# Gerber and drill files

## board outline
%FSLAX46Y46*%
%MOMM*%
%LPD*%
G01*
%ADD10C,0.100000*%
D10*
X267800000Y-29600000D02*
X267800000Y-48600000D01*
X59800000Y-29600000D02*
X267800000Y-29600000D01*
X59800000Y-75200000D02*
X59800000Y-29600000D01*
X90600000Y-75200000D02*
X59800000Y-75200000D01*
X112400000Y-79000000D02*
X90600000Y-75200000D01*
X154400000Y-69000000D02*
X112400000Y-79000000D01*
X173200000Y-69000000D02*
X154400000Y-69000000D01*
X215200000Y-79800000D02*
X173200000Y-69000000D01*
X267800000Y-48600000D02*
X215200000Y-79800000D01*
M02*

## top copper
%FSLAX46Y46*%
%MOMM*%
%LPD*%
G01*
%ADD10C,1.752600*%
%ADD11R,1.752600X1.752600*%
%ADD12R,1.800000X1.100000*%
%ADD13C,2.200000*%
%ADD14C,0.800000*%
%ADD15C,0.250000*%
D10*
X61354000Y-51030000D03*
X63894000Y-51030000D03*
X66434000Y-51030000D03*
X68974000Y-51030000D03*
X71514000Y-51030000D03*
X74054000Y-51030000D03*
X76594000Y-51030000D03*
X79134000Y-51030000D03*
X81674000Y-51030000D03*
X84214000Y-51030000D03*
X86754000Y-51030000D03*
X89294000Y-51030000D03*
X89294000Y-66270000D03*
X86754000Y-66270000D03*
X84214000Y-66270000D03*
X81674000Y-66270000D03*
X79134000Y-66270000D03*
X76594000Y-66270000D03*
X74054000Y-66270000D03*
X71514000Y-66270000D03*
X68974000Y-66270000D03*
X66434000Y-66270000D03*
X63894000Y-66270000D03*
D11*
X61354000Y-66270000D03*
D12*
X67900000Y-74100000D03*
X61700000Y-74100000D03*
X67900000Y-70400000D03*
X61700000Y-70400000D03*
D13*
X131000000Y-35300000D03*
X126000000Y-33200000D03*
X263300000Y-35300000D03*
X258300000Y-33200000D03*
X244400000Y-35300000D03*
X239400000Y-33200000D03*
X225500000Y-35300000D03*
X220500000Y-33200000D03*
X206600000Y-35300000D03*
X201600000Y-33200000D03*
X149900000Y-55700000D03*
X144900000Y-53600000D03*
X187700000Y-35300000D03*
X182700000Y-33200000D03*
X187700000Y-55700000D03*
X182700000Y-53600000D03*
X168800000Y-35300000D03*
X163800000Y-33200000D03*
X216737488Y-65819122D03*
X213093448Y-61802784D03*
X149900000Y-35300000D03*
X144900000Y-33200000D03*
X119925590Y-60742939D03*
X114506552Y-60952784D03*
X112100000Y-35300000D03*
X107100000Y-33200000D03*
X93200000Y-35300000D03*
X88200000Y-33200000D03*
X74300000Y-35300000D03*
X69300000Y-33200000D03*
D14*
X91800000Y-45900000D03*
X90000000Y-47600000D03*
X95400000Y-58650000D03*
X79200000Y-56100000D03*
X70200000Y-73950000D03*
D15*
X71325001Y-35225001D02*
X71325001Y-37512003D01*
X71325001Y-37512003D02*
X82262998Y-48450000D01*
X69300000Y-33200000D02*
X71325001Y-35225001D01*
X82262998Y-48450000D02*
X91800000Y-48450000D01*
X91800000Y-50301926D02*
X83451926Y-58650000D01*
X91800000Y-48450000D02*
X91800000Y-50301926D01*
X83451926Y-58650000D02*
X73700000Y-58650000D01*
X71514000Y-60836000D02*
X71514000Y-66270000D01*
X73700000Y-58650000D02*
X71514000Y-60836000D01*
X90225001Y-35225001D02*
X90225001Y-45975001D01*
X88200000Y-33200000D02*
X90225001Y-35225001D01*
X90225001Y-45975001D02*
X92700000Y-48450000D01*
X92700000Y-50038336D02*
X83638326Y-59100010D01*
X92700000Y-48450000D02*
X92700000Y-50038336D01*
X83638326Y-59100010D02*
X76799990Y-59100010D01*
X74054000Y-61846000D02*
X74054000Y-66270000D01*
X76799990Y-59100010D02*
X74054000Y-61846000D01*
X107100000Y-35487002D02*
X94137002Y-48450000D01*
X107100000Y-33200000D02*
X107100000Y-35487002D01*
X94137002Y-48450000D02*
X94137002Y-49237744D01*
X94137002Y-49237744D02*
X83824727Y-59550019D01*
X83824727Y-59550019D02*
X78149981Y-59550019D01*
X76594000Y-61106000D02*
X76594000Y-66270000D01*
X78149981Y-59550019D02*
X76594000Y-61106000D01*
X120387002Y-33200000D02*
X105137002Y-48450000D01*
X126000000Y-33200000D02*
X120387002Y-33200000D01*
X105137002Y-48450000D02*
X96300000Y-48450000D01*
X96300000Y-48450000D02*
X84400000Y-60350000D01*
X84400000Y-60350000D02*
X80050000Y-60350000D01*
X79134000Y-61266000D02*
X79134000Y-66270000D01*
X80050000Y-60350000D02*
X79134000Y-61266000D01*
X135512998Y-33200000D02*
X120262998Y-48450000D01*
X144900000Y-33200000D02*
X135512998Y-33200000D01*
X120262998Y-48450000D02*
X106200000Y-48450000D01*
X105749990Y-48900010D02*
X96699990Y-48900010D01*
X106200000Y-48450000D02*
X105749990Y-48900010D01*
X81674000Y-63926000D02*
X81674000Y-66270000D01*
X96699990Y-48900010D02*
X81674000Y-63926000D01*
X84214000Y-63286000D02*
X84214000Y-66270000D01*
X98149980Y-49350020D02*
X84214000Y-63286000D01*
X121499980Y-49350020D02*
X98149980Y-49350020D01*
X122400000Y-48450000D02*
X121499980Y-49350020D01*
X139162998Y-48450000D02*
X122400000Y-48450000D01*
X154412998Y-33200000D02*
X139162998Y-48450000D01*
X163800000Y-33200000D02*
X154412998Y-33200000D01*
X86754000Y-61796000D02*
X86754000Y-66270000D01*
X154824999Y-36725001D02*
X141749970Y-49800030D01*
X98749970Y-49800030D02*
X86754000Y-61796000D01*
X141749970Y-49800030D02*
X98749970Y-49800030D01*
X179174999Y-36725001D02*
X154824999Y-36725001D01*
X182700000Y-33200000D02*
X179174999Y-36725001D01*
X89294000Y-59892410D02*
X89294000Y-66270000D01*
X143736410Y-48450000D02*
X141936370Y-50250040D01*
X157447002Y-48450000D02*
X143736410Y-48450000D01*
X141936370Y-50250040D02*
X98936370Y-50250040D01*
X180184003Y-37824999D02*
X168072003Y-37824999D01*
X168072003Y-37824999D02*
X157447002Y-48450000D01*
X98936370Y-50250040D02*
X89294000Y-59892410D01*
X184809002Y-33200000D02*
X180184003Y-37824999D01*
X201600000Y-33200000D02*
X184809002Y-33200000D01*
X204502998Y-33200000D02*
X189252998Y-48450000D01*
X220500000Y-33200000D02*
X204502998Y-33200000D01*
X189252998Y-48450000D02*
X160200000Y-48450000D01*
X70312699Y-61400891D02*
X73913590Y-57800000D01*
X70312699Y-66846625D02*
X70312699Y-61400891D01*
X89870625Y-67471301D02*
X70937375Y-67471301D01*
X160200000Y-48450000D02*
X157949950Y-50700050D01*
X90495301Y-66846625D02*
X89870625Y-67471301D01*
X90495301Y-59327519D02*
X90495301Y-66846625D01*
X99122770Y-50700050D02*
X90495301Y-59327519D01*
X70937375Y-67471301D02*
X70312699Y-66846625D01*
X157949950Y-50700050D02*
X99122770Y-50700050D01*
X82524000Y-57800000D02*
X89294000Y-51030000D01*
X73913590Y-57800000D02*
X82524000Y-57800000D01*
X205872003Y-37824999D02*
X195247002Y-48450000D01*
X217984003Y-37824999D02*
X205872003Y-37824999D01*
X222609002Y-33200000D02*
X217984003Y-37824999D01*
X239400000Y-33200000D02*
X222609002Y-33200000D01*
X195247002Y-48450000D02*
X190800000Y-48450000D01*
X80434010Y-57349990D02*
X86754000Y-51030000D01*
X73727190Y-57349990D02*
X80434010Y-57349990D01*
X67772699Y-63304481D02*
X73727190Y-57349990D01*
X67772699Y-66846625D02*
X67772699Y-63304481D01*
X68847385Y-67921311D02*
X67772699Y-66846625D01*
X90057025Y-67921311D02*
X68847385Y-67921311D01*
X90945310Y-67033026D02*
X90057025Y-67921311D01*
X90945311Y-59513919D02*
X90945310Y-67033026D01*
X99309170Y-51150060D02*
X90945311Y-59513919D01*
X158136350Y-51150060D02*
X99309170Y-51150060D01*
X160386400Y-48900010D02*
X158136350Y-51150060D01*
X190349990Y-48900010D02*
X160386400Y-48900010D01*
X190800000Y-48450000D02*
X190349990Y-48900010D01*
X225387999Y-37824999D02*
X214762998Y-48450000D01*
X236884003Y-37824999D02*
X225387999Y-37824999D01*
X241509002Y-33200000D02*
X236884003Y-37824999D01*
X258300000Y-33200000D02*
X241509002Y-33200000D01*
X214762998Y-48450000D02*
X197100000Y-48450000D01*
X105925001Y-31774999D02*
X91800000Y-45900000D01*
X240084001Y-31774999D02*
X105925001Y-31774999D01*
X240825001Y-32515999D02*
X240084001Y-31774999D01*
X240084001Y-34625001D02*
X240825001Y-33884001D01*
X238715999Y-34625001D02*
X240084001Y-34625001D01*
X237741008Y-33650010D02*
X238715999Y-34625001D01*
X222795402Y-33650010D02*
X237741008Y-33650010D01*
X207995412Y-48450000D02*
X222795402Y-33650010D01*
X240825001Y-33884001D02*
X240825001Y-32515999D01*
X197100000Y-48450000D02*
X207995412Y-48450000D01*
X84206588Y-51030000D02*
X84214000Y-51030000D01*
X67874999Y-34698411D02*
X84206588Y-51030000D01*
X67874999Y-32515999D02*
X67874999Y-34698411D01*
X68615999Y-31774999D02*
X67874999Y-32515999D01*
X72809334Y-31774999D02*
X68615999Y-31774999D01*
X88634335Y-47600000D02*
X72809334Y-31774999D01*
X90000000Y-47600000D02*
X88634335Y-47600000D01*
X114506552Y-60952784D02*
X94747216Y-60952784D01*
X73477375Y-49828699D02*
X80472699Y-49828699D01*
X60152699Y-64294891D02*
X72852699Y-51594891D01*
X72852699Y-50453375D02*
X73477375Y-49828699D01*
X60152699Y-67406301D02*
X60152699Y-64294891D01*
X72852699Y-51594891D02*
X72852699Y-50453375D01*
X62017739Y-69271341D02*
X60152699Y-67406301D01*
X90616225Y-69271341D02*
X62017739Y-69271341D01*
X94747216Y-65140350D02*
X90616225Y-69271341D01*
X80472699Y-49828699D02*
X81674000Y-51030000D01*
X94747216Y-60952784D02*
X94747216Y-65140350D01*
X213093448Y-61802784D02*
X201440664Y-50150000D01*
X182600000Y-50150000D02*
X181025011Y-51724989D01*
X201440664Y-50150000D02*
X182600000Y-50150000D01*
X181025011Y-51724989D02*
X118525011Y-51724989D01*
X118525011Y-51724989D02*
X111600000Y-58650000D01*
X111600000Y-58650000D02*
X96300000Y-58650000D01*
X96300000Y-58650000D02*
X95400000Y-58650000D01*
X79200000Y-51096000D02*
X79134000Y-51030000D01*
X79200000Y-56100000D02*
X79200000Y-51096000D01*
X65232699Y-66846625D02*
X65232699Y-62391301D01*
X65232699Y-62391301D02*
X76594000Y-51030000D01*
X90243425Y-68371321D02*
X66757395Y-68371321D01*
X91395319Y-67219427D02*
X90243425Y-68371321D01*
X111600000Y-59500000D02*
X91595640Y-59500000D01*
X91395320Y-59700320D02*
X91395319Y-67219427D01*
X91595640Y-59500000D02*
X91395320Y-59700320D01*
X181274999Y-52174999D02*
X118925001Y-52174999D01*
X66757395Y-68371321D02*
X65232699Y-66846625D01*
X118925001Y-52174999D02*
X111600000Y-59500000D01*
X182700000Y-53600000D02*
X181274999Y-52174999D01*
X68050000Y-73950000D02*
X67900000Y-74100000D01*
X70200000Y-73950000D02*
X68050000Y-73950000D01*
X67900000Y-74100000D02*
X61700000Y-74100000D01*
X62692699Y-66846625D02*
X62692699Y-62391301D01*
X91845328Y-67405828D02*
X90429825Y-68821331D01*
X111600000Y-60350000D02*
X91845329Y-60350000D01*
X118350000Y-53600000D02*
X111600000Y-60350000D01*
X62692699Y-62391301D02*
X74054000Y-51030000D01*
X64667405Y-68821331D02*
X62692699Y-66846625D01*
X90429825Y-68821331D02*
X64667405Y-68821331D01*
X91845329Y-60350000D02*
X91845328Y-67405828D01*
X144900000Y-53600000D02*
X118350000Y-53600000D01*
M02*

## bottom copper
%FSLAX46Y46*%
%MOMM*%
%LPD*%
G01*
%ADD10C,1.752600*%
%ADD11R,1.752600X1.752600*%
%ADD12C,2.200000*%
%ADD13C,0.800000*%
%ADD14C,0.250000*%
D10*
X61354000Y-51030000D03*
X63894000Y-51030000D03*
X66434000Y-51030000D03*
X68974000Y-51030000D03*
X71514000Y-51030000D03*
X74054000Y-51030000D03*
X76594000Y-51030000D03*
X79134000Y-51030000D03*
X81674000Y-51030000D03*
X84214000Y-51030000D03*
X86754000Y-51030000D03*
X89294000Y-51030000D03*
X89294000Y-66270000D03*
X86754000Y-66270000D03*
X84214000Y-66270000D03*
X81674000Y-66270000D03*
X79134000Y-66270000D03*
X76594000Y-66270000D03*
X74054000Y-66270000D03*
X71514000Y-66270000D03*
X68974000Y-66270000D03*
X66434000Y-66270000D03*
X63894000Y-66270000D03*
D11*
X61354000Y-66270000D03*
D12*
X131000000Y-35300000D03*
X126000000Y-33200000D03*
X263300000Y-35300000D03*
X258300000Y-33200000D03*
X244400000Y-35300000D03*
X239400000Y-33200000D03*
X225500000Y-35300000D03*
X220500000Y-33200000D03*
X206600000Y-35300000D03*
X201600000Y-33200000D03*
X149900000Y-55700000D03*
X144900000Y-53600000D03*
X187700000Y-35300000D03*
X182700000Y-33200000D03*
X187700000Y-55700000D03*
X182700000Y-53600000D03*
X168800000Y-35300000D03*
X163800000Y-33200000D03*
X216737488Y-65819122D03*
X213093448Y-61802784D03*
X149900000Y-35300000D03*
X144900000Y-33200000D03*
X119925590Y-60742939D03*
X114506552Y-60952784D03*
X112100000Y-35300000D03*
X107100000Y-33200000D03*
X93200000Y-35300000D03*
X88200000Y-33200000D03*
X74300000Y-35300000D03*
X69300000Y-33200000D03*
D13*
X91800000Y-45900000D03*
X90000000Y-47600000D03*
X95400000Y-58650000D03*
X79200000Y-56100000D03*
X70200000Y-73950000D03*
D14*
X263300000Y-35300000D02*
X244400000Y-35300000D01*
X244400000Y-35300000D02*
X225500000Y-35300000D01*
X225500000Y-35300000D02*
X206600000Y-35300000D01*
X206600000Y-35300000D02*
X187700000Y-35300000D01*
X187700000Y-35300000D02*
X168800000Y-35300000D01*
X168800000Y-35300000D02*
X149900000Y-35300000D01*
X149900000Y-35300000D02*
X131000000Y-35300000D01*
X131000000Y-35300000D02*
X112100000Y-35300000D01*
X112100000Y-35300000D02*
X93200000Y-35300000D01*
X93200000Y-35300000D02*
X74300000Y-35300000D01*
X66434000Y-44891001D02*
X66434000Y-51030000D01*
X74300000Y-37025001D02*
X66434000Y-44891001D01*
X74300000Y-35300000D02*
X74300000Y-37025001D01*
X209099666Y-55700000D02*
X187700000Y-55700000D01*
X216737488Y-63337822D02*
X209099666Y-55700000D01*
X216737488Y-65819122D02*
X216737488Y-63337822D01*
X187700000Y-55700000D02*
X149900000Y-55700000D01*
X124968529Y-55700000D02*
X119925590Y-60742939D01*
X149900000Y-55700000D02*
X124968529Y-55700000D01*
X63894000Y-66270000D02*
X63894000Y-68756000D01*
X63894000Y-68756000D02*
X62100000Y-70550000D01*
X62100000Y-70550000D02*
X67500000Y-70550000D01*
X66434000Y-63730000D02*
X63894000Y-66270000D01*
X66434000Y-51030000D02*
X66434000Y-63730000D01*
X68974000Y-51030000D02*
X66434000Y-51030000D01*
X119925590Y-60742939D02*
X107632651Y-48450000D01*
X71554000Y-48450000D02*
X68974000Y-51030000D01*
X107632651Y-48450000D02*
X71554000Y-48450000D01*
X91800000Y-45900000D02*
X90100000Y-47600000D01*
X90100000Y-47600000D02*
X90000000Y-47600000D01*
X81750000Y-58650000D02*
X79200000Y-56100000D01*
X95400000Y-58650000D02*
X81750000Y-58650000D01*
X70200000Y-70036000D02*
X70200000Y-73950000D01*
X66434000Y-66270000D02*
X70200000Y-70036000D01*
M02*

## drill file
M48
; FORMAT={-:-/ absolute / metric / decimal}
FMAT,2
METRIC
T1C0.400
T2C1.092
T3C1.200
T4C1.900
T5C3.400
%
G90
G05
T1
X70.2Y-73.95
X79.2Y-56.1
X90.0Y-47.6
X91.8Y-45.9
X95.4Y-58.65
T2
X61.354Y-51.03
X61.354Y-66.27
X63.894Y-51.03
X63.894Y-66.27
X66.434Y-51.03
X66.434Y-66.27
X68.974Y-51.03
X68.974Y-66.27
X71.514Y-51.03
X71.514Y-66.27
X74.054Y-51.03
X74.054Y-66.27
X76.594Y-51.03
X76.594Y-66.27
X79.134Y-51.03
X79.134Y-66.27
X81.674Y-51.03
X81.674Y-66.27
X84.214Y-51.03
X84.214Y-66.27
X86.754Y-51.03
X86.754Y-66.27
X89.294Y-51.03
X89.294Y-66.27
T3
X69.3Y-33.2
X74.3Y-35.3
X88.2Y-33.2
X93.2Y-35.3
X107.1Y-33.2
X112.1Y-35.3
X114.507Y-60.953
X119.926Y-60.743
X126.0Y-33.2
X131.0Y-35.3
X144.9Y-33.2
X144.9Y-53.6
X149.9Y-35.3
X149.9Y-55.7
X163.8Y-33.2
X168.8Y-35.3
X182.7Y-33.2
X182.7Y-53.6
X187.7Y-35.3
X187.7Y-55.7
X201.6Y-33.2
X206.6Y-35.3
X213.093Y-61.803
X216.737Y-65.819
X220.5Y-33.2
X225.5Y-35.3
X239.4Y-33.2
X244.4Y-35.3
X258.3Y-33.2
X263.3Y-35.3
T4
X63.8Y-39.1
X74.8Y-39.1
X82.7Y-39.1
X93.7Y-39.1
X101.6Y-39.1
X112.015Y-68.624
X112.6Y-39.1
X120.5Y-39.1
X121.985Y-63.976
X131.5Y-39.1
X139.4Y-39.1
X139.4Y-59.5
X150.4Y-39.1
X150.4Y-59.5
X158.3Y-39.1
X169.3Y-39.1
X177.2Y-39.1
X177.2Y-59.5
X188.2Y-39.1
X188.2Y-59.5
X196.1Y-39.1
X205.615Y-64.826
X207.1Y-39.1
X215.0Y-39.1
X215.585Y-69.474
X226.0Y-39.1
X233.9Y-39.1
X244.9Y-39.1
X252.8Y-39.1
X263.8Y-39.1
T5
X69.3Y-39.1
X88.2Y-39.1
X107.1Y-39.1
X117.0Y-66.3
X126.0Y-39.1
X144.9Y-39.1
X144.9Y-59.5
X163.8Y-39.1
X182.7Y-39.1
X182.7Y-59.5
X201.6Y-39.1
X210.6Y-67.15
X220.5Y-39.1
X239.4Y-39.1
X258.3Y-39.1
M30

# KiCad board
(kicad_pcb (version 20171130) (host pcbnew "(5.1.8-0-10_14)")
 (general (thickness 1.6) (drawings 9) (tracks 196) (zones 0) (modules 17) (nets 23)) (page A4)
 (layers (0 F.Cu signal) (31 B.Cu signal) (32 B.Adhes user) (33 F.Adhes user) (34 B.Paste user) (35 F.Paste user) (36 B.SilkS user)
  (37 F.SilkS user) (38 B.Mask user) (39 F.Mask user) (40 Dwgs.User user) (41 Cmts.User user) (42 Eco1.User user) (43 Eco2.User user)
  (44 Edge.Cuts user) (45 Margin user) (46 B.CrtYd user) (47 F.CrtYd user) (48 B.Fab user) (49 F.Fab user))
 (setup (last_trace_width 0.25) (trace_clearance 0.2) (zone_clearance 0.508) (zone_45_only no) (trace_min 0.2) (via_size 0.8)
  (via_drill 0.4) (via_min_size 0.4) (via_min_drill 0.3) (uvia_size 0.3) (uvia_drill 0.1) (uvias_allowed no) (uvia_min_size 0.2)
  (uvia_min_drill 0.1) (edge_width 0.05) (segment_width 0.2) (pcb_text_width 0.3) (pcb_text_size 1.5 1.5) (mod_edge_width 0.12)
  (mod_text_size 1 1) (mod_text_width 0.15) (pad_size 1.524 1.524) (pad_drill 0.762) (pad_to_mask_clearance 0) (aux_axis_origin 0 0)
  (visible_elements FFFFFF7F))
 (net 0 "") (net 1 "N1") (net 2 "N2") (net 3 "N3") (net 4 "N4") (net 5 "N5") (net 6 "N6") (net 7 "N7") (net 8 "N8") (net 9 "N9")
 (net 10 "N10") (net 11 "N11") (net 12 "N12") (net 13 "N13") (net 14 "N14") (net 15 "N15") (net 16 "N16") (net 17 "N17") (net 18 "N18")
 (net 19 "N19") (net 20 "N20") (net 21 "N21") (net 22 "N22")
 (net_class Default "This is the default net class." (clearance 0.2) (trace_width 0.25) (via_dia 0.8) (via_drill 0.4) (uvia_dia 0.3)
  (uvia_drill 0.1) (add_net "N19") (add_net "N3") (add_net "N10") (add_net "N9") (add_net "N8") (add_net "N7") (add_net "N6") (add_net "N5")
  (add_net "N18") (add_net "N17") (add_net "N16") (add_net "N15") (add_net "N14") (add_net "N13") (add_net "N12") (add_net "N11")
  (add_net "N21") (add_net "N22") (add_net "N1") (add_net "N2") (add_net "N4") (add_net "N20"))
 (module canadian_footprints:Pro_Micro (layer F.Cu) (at 73.8 58.65 90)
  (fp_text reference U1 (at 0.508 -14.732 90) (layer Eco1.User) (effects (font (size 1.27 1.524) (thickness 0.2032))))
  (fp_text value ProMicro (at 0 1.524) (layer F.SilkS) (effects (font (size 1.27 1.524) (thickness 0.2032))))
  (pad 13 thru_hole circle (at 7.62 -12.446) (size 1.7526 1.7526) (drill 1.0922) (layers *.Cu *.SilkS *.Mask) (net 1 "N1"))
  (pad 14 thru_hole circle (at 7.62 -9.906) (size 1.7526 1.7526) (drill 1.0922) (layers *.Cu *.SilkS *.Mask) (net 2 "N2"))
  (pad 15 thru_hole circle (at 7.62 -7.366) (size 1.7526 1.7526) (drill 1.0922) (layers *.Cu *.SilkS *.Mask) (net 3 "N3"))
  (pad 16 thru_hole circle (at 7.62 -4.826) (size 1.7526 1.7526) (drill 1.0922) (layers *.Cu *.SilkS *.Mask) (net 3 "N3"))
  (pad 17 thru_hole circle (at 7.62 -2.286) (size 1.7526 1.7526) (drill 1.0922) (layers *.Cu *.SilkS *.Mask) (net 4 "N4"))
  (pad 18 thru_hole circle (at 7.62 0.254) (size 1.7526 1.7526) (drill 1.0922) (layers *.Cu *.SilkS *.Mask) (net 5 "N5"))
  (pad 19 thru_hole circle (at 7.62 2.794) (size 1.7526 1.7526) (drill 1.0922) (layers *.Cu *.SilkS *.Mask) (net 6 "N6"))
  (pad 20 thru_hole circle (at 7.62 5.334) (size 1.7526 1.7526) (drill 1.0922) (layers *.Cu *.SilkS *.Mask) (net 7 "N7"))
  (pad 21 thru_hole circle (at 7.62 7.874) (size 1.7526 1.7526) (drill 1.0922) (layers *.Cu *.SilkS *.Mask) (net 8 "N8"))
  (pad 22 thru_hole circle (at 7.62 10.414) (size 1.7526 1.7526) (drill 1.0922) (layers *.Cu *.SilkS *.Mask) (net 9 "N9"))
  (pad 23 thru_hole circle (at 7.62 12.954) (size 1.7526 1.7526) (drill 1.0922) (layers *.Cu *.SilkS *.Mask) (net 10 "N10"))
  (pad 24 thru_hole circle (at 7.62 15.494) (size 1.7526 1.7526) (drill 1.0922) (layers *.Cu *.SilkS *.Mask) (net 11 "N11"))
  (pad 12 thru_hole circle (at -7.62 15.494) (size 1.7526 1.7526) (drill 1.0922) (layers *.Cu *.SilkS *.Mask) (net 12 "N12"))
  (pad 11 thru_hole circle (at -7.62 12.954) (size 1.7526 1.7526) (drill 1.0922) (layers *.Cu *.SilkS *.Mask) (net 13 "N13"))
  (pad 10 thru_hole circle (at -7.62 10.414) (size 1.7526 1.7526) (drill 1.0922) (layers *.Cu *.SilkS *.Mask) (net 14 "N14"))
  (pad 9 thru_hole circle (at -7.62 7.874) (size 1.7526 1.7526) (drill 1.0922) (layers *.Cu *.SilkS *.Mask) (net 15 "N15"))
  (pad 8 thru_hole circle (at -7.62 5.334) (size 1.7526 1.7526) (drill 1.0922) (layers *.Cu *.SilkS *.Mask) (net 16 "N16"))
  (pad 7 thru_hole circle (at -7.62 2.794) (size 1.7526 1.7526) (drill 1.0922) (layers *.Cu *.SilkS *.Mask) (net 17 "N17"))
  (pad 6 thru_hole circle (at -7.62 0.254) (size 1.7526 1.7526) (drill 1.0922) (layers *.Cu *.SilkS *.Mask) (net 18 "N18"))
  (pad 5 thru_hole circle (at -7.62 -2.286) (size 1.7526 1.7526) (drill 1.0922) (layers *.Cu *.SilkS *.Mask) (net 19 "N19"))
  (pad 4 thru_hole circle (at -7.62 -4.826) (size 1.7526 1.7526) (drill 1.0922) (layers *.Cu *.SilkS *.Mask) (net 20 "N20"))
  (pad 3 thru_hole circle (at -7.62 -7.366) (size 1.7526 1.7526) (drill 1.0922) (layers *.Cu *.SilkS *.Mask) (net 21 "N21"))
  (pad 2 thru_hole circle (at -7.62 -9.906) (size 1.7526 1.7526) (drill 1.0922) (layers *.Cu *.SilkS *.Mask) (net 3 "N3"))
  (pad 1 thru_hole rect (at -7.62 -12.446) (size 1.7526 1.7526) (drill 1.0922) (layers *.Cu *.SilkS *.Mask) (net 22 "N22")))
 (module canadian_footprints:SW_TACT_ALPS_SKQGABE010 (layer F.Cu) (at 64.8 72.25)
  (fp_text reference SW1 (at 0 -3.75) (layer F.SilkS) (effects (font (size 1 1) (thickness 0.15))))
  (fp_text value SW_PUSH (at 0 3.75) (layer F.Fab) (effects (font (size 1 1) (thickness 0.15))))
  (pad 2 smd rect (at 3.1 1.85) (size 1.8 1.1) (layers F.Cu F.Paste F.Mask) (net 21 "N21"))
  (pad 2 smd rect (at -3.1 1.85) (size 1.8 1.1) (layers F.Cu F.Paste F.Mask) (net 21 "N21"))
  (pad 1 smd rect (at 3.1 -1.85) (size 1.8 1.1) (layers F.Cu F.Paste F.Mask) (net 3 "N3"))
  (pad 1 smd rect (at -3.1 -1.85) (size 1.8 1.1) (layers F.Cu F.Paste F.Mask) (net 3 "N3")))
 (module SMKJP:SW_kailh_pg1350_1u (layer F.Cu) (at 126 39.1)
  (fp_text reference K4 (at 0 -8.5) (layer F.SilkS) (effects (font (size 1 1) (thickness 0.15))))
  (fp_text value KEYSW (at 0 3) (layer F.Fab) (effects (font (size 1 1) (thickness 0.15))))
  (pad 2 thru_hole circle (at 5 -3.8) (size 2.2 2.2) (drill 1.2) (layers *.Cu *.Mask) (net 3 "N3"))
  (pad 1 thru_hole circle (at 0 -5.9) (size 2.2 2.2) (drill 1.2) (layers *.Cu *.Mask) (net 16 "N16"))
  (pad "" np_thru_hole circle (at 5.5 0) (size 1.9 1.9) (drill 1.9) (layers *.Cu *.Mask))
  (pad "" np_thru_hole circle (at -5.5 0) (size 1.9 1.9) (drill 1.9) (layers *.Cu *.Mask))
  (pad "" np_thru_hole circle (at 0 0) (size 3.4 3.4) (drill 3.4) (layers *.Cu *.Mask)))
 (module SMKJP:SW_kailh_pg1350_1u (layer F.Cu) (at 258.3 39.1)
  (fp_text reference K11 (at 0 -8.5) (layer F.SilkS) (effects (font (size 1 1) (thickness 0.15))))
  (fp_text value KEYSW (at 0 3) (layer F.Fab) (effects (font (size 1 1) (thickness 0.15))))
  (pad 2 thru_hole circle (at 5 -3.8) (size 2.2 2.2) (drill 1.2) (layers *.Cu *.Mask) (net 3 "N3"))
  (pad 1 thru_hole circle (at 0 -5.9) (size 2.2 2.2) (drill 1.2) (layers *.Cu *.Mask) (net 9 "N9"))
  (pad "" np_thru_hole circle (at 5.5 0) (size 1.9 1.9) (drill 1.9) (layers *.Cu *.Mask))
  (pad "" np_thru_hole circle (at -5.5 0) (size 1.9 1.9) (drill 1.9) (layers *.Cu *.Mask))
  (pad "" np_thru_hole circle (at 0 0) (size 3.4 3.4) (drill 3.4) (layers *.Cu *.Mask)))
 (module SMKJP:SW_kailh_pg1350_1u (layer F.Cu) (at 239.4 39.1)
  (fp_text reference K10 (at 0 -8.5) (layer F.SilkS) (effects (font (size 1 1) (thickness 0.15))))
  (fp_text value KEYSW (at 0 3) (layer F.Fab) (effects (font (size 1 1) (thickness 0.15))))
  (pad 2 thru_hole circle (at 5 -3.8) (size 2.2 2.2) (drill 1.2) (layers *.Cu *.Mask) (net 3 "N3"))
  (pad 1 thru_hole circle (at 0 -5.9) (size 2.2 2.2) (drill 1.2) (layers *.Cu *.Mask) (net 10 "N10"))
  (pad "" np_thru_hole circle (at 5.5 0) (size 1.9 1.9) (drill 1.9) (layers *.Cu *.Mask))
  (pad "" np_thru_hole circle (at -5.5 0) (size 1.9 1.9) (drill 1.9) (layers *.Cu *.Mask))
  (pad "" np_thru_hole circle (at 0 0) (size 3.4 3.4) (drill 3.4) (layers *.Cu *.Mask)))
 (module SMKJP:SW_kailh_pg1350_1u (layer F.Cu) (at 220.5 39.1)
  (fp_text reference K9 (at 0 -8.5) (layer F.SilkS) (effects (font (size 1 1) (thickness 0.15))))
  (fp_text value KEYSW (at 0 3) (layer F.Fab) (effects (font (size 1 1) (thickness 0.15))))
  (pad 2 thru_hole circle (at 5 -3.8) (size 2.2 2.2) (drill 1.2) (layers *.Cu *.Mask) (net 3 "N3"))
  (pad 1 thru_hole circle (at 0 -5.9) (size 2.2 2.2) (drill 1.2) (layers *.Cu *.Mask) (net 11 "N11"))
  (pad "" np_thru_hole circle (at 5.5 0) (size 1.9 1.9) (drill 1.9) (layers *.Cu *.Mask))
  (pad "" np_thru_hole circle (at -5.5 0) (size 1.9 1.9) (drill 1.9) (layers *.Cu *.Mask))
  (pad "" np_thru_hole circle (at 0 0) (size 3.4 3.4) (drill 3.4) (layers *.Cu *.Mask)))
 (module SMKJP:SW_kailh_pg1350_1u (layer F.Cu) (at 201.6 39.1)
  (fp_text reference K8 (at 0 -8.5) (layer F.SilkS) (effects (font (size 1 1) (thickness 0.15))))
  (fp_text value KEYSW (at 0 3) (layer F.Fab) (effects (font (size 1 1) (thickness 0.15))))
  (pad 2 thru_hole circle (at 5 -3.8) (size 2.2 2.2) (drill 1.2) (layers *.Cu *.Mask) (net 3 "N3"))
  (pad 1 thru_hole circle (at 0 -5.9) (size 2.2 2.2) (drill 1.2) (layers *.Cu *.Mask) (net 12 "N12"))
  (pad "" np_thru_hole circle (at 5.5 0) (size 1.9 1.9) (drill 1.9) (layers *.Cu *.Mask))
  (pad "" np_thru_hole circle (at -5.5 0) (size 1.9 1.9) (drill 1.9) (layers *.Cu *.Mask))
  (pad "" np_thru_hole circle (at 0 0) (size 3.4 3.4) (drill 3.4) (layers *.Cu *.Mask)))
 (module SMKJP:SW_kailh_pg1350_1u (layer F.Cu) (at 144.9 59.5)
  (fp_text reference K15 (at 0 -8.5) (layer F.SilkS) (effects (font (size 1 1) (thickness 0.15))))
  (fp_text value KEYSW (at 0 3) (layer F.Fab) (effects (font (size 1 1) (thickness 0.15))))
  (pad 2 thru_hole circle (at 5 -3.8) (size 2.2 2.2) (drill 1.2) (layers *.Cu *.Mask) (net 3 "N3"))
  (pad 1 thru_hole circle (at 0 -5.9) (size 2.2 2.2) (drill 1.2) (layers *.Cu *.Mask) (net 5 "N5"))
  (pad "" np_thru_hole circle (at 5.5 0) (size 1.9 1.9) (drill 1.9) (layers *.Cu *.Mask))
  (pad "" np_thru_hole circle (at -5.5 0) (size 1.9 1.9) (drill 1.9) (layers *.Cu *.Mask))
  (pad "" np_thru_hole circle (at 0 0) (size 3.4 3.4) (drill 3.4) (layers *.Cu *.Mask)))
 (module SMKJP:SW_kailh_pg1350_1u (layer F.Cu) (at 182.7 39.1)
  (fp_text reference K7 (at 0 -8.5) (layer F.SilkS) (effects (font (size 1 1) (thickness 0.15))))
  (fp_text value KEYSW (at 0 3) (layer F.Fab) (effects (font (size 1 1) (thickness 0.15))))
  (pad 2 thru_hole circle (at 5 -3.8) (size 2.2 2.2) (drill 1.2) (layers *.Cu *.Mask) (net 3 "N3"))
  (pad 1 thru_hole circle (at 0 -5.9) (size 2.2 2.2) (drill 1.2) (layers *.Cu *.Mask) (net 13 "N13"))
  (pad "" np_thru_hole circle (at 5.5 0) (size 1.9 1.9) (drill 1.9) (layers *.Cu *.Mask))
  (pad "" np_thru_hole circle (at -5.5 0) (size 1.9 1.9) (drill 1.9) (layers *.Cu *.Mask))
  (pad "" np_thru_hole circle (at 0 0) (size 3.4 3.4) (drill 3.4) (layers *.Cu *.Mask)))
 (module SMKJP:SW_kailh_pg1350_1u (layer F.Cu) (at 182.7 59.5)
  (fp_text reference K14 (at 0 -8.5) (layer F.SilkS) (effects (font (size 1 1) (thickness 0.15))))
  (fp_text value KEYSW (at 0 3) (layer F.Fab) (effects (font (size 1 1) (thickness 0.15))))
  (pad 2 thru_hole circle (at 5 -3.8) (size 2.2 2.2) (drill 1.2) (layers *.Cu *.Mask) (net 3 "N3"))
  (pad 1 thru_hole circle (at 0 -5.9) (size 2.2 2.2) (drill 1.2) (layers *.Cu *.Mask) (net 6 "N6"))
  (pad "" np_thru_hole circle (at 5.5 0) (size 1.9 1.9) (drill 1.9) (layers *.Cu *.Mask))
  (pad "" np_thru_hole circle (at -5.5 0) (size 1.9 1.9) (drill 1.9) (layers *.Cu *.Mask))
  (pad "" np_thru_hole circle (at 0 0) (size 3.4 3.4) (drill 3.4) (layers *.Cu *.Mask)))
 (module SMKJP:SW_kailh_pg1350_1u (layer F.Cu) (at 163.8 39.1)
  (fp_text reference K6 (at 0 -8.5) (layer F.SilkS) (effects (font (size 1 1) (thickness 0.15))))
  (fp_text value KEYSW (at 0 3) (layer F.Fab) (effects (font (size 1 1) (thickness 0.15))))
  (pad 2 thru_hole circle (at 5 -3.8) (size 2.2 2.2) (drill 1.2) (layers *.Cu *.Mask) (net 3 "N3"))
  (pad 1 thru_hole circle (at 0 -5.9) (size 2.2 2.2) (drill 1.2) (layers *.Cu *.Mask) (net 14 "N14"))
  (pad "" np_thru_hole circle (at 5.5 0) (size 1.9 1.9) (drill 1.9) (layers *.Cu *.Mask))
  (pad "" np_thru_hole circle (at -5.5 0) (size 1.9 1.9) (drill 1.9) (layers *.Cu *.Mask))
  (pad "" np_thru_hole circle (at 0 0) (size 3.4 3.4) (drill 3.4) (layers *.Cu *.Mask)))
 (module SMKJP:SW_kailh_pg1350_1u (layer F.Cu) (at 210.6 67.15 335)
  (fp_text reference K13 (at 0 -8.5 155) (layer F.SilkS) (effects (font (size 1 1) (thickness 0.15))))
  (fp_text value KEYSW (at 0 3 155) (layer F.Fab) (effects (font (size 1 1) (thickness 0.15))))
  (pad 2 thru_hole circle (at 5 -3.8 335) (size 2.2 2.2) (drill 1.2) (layers *.Cu *.Mask) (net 3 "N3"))
  (pad 1 thru_hole circle (at 0 -5.9 335) (size 2.2 2.2) (drill 1.2) (layers *.Cu *.Mask) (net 7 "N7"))
  (pad "" np_thru_hole circle (at 5.5 0 335) (size 1.9 1.9) (drill 1.9) (layers *.Cu *.Mask))
  (pad "" np_thru_hole circle (at -5.5 0 335) (size 1.9 1.9) (drill 1.9) (layers *.Cu *.Mask))
  (pad "" np_thru_hole circle (at 0 0 335) (size 3.4 3.4) (drill 3.4) (layers *.Cu *.Mask)))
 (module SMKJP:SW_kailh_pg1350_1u (layer F.Cu) (at 144.9 39.1)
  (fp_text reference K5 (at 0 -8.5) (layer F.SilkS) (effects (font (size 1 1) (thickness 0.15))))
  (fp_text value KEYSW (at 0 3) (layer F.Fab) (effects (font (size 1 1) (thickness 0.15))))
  (pad 2 thru_hole circle (at 5 -3.8) (size 2.2 2.2) (drill 1.2) (layers *.Cu *.Mask) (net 3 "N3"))
  (pad 1 thru_hole circle (at 0 -5.9) (size 2.2 2.2) (drill 1.2) (layers *.Cu *.Mask) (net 15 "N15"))
  (pad "" np_thru_hole circle (at 5.5 0) (size 1.9 1.9) (drill 1.9) (layers *.Cu *.Mask))
  (pad "" np_thru_hole circle (at -5.5 0) (size 1.9 1.9) (drill 1.9) (layers *.Cu *.Mask))
  (pad "" np_thru_hole circle (at 0 0) (size 3.4 3.4) (drill 3.4) (layers *.Cu *.Mask)))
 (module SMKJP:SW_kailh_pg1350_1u (layer F.Cu) (at 117 66.3 25)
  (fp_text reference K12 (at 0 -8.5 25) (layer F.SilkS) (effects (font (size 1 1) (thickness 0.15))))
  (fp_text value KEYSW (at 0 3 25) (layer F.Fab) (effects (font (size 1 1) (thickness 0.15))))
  (pad 2 thru_hole circle (at 5 -3.8 25) (size 2.2 2.2) (drill 1.2) (layers *.Cu *.Mask) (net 3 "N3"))
  (pad 1 thru_hole circle (at 0 -5.9 25) (size 2.2 2.2) (drill 1.2) (layers *.Cu *.Mask) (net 8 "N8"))
  (pad "" np_thru_hole circle (at 5.5 0 25) (size 1.9 1.9) (drill 1.9) (layers *.Cu *.Mask))
  (pad "" np_thru_hole circle (at -5.5 0 25) (size 1.9 1.9) (drill 1.9) (layers *.Cu *.Mask))
  (pad "" np_thru_hole circle (at 0 0 25) (size 3.4 3.4) (drill 3.4) (layers *.Cu *.Mask)))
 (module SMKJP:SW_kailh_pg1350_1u (layer F.Cu) (at 107.1 39.1)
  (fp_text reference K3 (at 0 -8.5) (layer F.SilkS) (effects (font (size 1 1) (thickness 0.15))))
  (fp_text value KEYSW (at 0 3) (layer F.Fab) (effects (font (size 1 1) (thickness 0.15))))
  (pad 2 thru_hole circle (at 5 -3.8) (size 2.2 2.2) (drill 1.2) (layers *.Cu *.Mask) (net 3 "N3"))
  (pad 1 thru_hole circle (at 0 -5.9) (size 2.2 2.2) (drill 1.2) (layers *.Cu *.Mask) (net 17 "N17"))
  (pad "" np_thru_hole circle (at 5.5 0) (size 1.9 1.9) (drill 1.9) (layers *.Cu *.Mask))
  (pad "" np_thru_hole circle (at -5.5 0) (size 1.9 1.9) (drill 1.9) (layers *.Cu *.Mask))
  (pad "" np_thru_hole circle (at 0 0) (size 3.4 3.4) (drill 3.4) (layers *.Cu *.Mask)))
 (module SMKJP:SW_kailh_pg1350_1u (layer F.Cu) (at 88.2 39.1)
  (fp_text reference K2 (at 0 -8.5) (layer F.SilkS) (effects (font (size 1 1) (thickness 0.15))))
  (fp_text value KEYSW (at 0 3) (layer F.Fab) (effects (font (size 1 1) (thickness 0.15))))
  (pad 2 thru_hole circle (at 5 -3.8) (size 2.2 2.2) (drill 1.2) (layers *.Cu *.Mask) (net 3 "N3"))
  (pad 1 thru_hole circle (at 0 -5.9) (size 2.2 2.2) (drill 1.2) (layers *.Cu *.Mask) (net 18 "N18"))
  (pad "" np_thru_hole circle (at 5.5 0) (size 1.9 1.9) (drill 1.9) (layers *.Cu *.Mask))
  (pad "" np_thru_hole circle (at -5.5 0) (size 1.9 1.9) (drill 1.9) (layers *.Cu *.Mask))
  (pad "" np_thru_hole circle (at 0 0) (size 3.4 3.4) (drill 3.4) (layers *.Cu *.Mask)))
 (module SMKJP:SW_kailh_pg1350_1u (layer F.Cu) (at 69.3 39.1)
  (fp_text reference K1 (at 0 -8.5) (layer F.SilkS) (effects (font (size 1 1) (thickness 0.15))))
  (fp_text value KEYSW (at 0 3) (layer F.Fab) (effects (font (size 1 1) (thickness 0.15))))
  (pad 2 thru_hole circle (at 5 -3.8) (size 2.2 2.2) (drill 1.2) (layers *.Cu *.Mask) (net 3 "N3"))
  (pad 1 thru_hole circle (at 0 -5.9) (size 2.2 2.2) (drill 1.2) (layers *.Cu *.Mask) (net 19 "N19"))
  (pad "" np_thru_hole circle (at 5.5 0) (size 1.9 1.9) (drill 1.9) (layers *.Cu *.Mask))
  (pad "" np_thru_hole circle (at -5.5 0) (size 1.9 1.9) (drill 1.9) (layers *.Cu *.Mask))
  (pad "" np_thru_hole circle (at 0 0) (size 3.4 3.4) (drill 3.4) (layers *.Cu *.Mask)))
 (gr_line (start 267.8 29.6) (end 267.8 48.6) (layer Edge.Cuts) (width 0.1))
 (gr_line (start 59.8 29.6) (end 267.8 29.6) (layer Edge.Cuts) (width 0.1))
 (gr_line (start 59.8 75.2) (end 59.8 29.6) (layer Edge.Cuts) (width 0.1))
 (gr_line (start 90.6 75.2) (end 59.8 75.2) (layer Edge.Cuts) (width 0.1))
 (gr_line (start 112.4 79) (end 90.6 75.2) (layer Edge.Cuts) (width 0.1))
 (gr_line (start 154.4 69) (end 112.4 79) (layer Edge.Cuts) (width 0.1))
 (gr_line (start 173.2 69) (end 154.4 69) (layer Edge.Cuts) (width 0.1))
 (gr_line (start 215.2 79.8) (end 173.2 69) (layer Edge.Cuts) (width 0.1))
 (gr_line (start 267.8 48.6) (end 215.2 79.8) (layer Edge.Cuts) (width 0.1))
 (segment (start 263.3 35.3) (end 244.4 35.3) (width 0.25) (layer B.Cu) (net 3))
 (segment (start 244.4 35.3) (end 225.5 35.3) (width 0.25) (layer B.Cu) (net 3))
 (segment (start 225.5 35.3) (end 206.6 35.3) (width 0.25) (layer B.Cu) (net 3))
 (segment (start 206.6 35.3) (end 187.7 35.3) (width 0.25) (layer B.Cu) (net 3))
 (segment (start 187.7 35.3) (end 168.8 35.3) (width 0.25) (layer B.Cu) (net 3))
 (segment (start 168.8 35.3) (end 149.9 35.3) (width 0.25) (layer B.Cu) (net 3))
 (segment (start 149.9 35.3) (end 131 35.3) (width 0.25) (layer B.Cu) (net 3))
 (segment (start 131 35.3) (end 112.1 35.3) (width 0.25) (layer B.Cu) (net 3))
 (segment (start 112.1 35.3) (end 93.2 35.3) (width 0.25) (layer B.Cu) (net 3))
 (segment (start 93.2 35.3) (end 74.3 35.3) (width 0.25) (layer B.Cu) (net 3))
 (segment (start 66.434 44.891001) (end 66.434 51.03) (width 0.25) (layer B.Cu) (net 3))
 (segment (start 74.3 37.025001) (end 66.434 44.891001) (width 0.25) (layer B.Cu) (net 3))
 (segment (start 74.3 35.3) (end 74.3 37.025001) (width 0.25) (layer B.Cu) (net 3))
 (segment (start 209.099666 55.7) (end 187.7 55.7) (width 0.25) (layer B.Cu) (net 3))
 (segment (start 216.737488 63.337822) (end 209.099666 55.7) (width 0.25) (layer B.Cu) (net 3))
 (segment (start 216.737488 65.819122) (end 216.737488 63.337822) (width 0.25) (layer B.Cu) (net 3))
 (segment (start 187.7 55.7) (end 149.9 55.7) (width 0.25) (layer B.Cu) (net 3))
 (segment (start 124.968529 55.7) (end 119.92559 60.742939) (width 0.25) (layer B.Cu) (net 3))
 (segment (start 149.9 55.7) (end 124.968529 55.7) (width 0.25) (layer B.Cu) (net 3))
 (segment (start 63.894 66.27) (end 63.894 68.756) (width 0.25) (layer B.Cu) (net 3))
 (segment (start 63.894 68.756) (end 62.1 70.55) (width 0.25) (layer B.Cu) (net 3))
 (segment (start 62.1 70.55) (end 67.5 70.55) (width 0.25) (layer B.Cu) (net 3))
 (segment (start 66.434 63.73) (end 63.894 66.27) (width 0.25) (layer B.Cu) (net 3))
 (segment (start 66.434 51.03) (end 66.434 63.73) (width 0.25) (layer B.Cu) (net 3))
 (segment (start 68.974 51.03) (end 66.434 51.03) (width 0.25) (layer B.Cu) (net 3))
 (segment (start 119.92559 60.742939) (end 107.632651 48.45) (width 0.25) (layer B.Cu) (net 3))
 (segment (start 71.554 48.45) (end 68.974 51.03) (width 0.25) (layer B.Cu) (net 3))
 (segment (start 107.632651 48.45) (end 71.554 48.45) (width 0.25) (layer B.Cu) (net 3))
 (segment (start 71.325001 35.225001) (end 71.325001 37.512003) (width 0.25) (layer F.Cu) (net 19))
 (segment (start 71.325001 37.512003) (end 82.262998 48.45) (width 0.25) (layer F.Cu) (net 19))
 (segment (start 69.3 33.2) (end 71.325001 35.225001) (width 0.25) (layer F.Cu) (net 19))
 (segment (start 82.262998 48.45) (end 91.8 48.45) (width 0.25) (layer F.Cu) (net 19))
 (segment (start 91.8 50.301926) (end 83.451926 58.65) (width 0.25) (layer F.Cu) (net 19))
 (segment (start 91.8 48.45) (end 91.8 50.301926) (width 0.25) (layer F.Cu) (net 19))
 (segment (start 83.451926 58.65) (end 73.7 58.65) (width 0.25) (layer F.Cu) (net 19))
 (segment (start 71.514 60.836) (end 71.514 66.27) (width 0.25) (layer F.Cu) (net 19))
 (segment (start 73.7 58.65) (end 71.514 60.836) (width 0.25) (layer F.Cu) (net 19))
 (segment (start 90.225001 35.225001) (end 90.225001 45.975001) (width 0.25) (layer F.Cu) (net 18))
 (segment (start 88.2 33.2) (end 90.225001 35.225001) (width 0.25) (layer F.Cu) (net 18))
 (segment (start 90.225001 45.975001) (end 92.7 48.45) (width 0.25) (layer F.Cu) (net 18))
 (segment (start 92.7 50.038336) (end 83.638326 59.10001) (width 0.25) (layer F.Cu) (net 18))
 (segment (start 92.7 48.45) (end 92.7 50.038336) (width 0.25) (layer F.Cu) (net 18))
 (segment (start 83.638326 59.10001) (end 76.79999 59.10001) (width 0.25) (layer F.Cu) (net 18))
 (segment (start 74.054 61.846) (end 74.054 66.27) (width 0.25) (layer F.Cu) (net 18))
 (segment (start 76.79999 59.10001) (end 74.054 61.846) (width 0.25) (layer F.Cu) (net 18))
 (segment (start 107.1 35.487002) (end 94.137002 48.45) (width 0.25) (layer F.Cu) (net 17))
 (segment (start 107.1 33.2) (end 107.1 35.487002) (width 0.25) (layer F.Cu) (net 17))
 (segment (start 94.137002 48.45) (end 94.137002 49.237744) (width 0.25) (layer F.Cu) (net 17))
 (segment (start 94.137002 49.237744) (end 83.824727 59.550019) (width 0.25) (layer F.Cu) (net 17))
 (segment (start 83.824727 59.550019) (end 78.149981 59.550019) (width 0.25) (layer F.Cu) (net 17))
 (segment (start 76.594 61.106) (end 76.594 66.27) (width 0.25) (layer F.Cu) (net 17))
 (segment (start 78.149981 59.550019) (end 76.594 61.106) (width 0.25) (layer F.Cu) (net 17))
 (segment (start 120.387002 33.2) (end 105.137002 48.45) (width 0.25) (layer F.Cu) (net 16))
 (segment (start 126 33.2) (end 120.387002 33.2) (width 0.25) (layer F.Cu) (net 16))
 (segment (start 105.137002 48.45) (end 96.3 48.45) (width 0.25) (layer F.Cu) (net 16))
 (segment (start 96.3 48.45) (end 84.4 60.35) (width 0.25) (layer F.Cu) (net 16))
 (segment (start 84.4 60.35) (end 80.05 60.35) (width 0.25) (layer F.Cu) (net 16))
 (segment (start 79.134 61.266) (end 79.134 66.27) (width 0.25) (layer F.Cu) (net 16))
 (segment (start 80.05 60.35) (end 79.134 61.266) (width 0.25) (layer F.Cu) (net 16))
 (segment (start 135.512998 33.2) (end 120.262998 48.45) (width 0.25) (layer F.Cu) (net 15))
 (segment (start 144.9 33.2) (end 135.512998 33.2) (width 0.25) (layer F.Cu) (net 15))
 (segment (start 120.262998 48.45) (end 106.2 48.45) (width 0.25) (layer F.Cu) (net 15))
 (segment (start 105.74999 48.90001) (end 96.69999 48.90001) (width 0.25) (layer F.Cu) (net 15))
 (segment (start 106.2 48.45) (end 105.74999 48.90001) (width 0.25) (layer F.Cu) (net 15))
 (segment (start 81.674 63.926) (end 81.674 66.27) (width 0.25) (layer F.Cu) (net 15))
 (segment (start 96.69999 48.90001) (end 81.674 63.926) (width 0.25) (layer F.Cu) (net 15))
 (segment (start 84.214 63.286) (end 84.214 66.27) (width 0.25) (layer F.Cu) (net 14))
 (segment (start 98.14998 49.35002) (end 84.214 63.286) (width 0.25) (layer F.Cu) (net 14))
 (segment (start 121.49998 49.35002) (end 98.14998 49.35002) (width 0.25) (layer F.Cu) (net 14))
 (segment (start 122.4 48.45) (end 121.49998 49.35002) (width 0.25) (layer F.Cu) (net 14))
 (segment (start 139.162998 48.45) (end 122.4 48.45) (width 0.25) (layer F.Cu) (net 14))
 (segment (start 154.412998 33.2) (end 139.162998 48.45) (width 0.25) (layer F.Cu) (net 14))
 (segment (start 163.8 33.2) (end 154.412998 33.2) (width 0.25) (layer F.Cu) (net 14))
 (segment (start 86.754 61.796) (end 86.754 66.27) (width 0.25) (layer F.Cu) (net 13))
 (segment (start 154.824999 36.725001) (end 141.74997 49.80003) (width 0.25) (layer F.Cu) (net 13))
 (segment (start 98.74997 49.80003) (end 86.754 61.796) (width 0.25) (layer F.Cu) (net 13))
 (segment (start 141.74997 49.80003) (end 98.74997 49.80003) (width 0.25) (layer F.Cu) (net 13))
 (segment (start 179.174999 36.725001) (end 154.824999 36.725001) (width 0.25) (layer F.Cu) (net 13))
 (segment (start 182.7 33.2) (end 179.174999 36.725001) (width 0.25) (layer F.Cu) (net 13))
 (segment (start 89.294 59.89241) (end 89.294 66.27) (width 0.25) (layer F.Cu) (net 12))
 (segment (start 143.73641 48.45) (end 141.93637 50.25004) (width 0.25) (layer F.Cu) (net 12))
 (segment (start 157.447002 48.45) (end 143.73641 48.45) (width 0.25) (layer F.Cu) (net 12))
 (segment (start 141.93637 50.25004) (end 98.93637 50.25004) (width 0.25) (layer F.Cu) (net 12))
 (segment (start 180.184003 37.824999) (end 168.072003 37.824999) (width 0.25) (layer F.Cu) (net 12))
 (segment (start 168.072003 37.824999) (end 157.447002 48.45) (width 0.25) (layer F.Cu) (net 12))
 (segment (start 98.93637 50.25004) (end 89.294 59.89241) (width 0.25) (layer F.Cu) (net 12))
 (segment (start 184.809002 33.2) (end 180.184003 37.824999) (width 0.25) (layer F.Cu) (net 12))
 (segment (start 201.6 33.2) (end 184.809002 33.2) (width 0.25) (layer F.Cu) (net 12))
 (segment (start 204.502998 33.2) (end 189.252998 48.45) (width 0.25) (layer F.Cu) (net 11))
 (segment (start 220.5 33.2) (end 204.502998 33.2) (width 0.25) (layer F.Cu) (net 11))
 (segment (start 189.252998 48.45) (end 160.2 48.45) (width 0.25) (layer F.Cu) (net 11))
 (segment (start 70.312699 61.400891) (end 73.91359 57.8) (width 0.25) (layer F.Cu) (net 11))
 (segment (start 70.312699 66.846625) (end 70.312699 61.400891) (width 0.25) (layer F.Cu) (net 11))
 (segment (start 89.870625 67.471301) (end 70.937375 67.471301) (width 0.25) (layer F.Cu) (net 11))
 (segment (start 160.2 48.45) (end 157.94995 50.70005) (width 0.25) (layer F.Cu) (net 11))
 (segment (start 90.495301 66.846625) (end 89.870625 67.471301) (width 0.25) (layer F.Cu) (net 11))
 (segment (start 90.495301 59.327519) (end 90.495301 66.846625) (width 0.25) (layer F.Cu) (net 11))
 (segment (start 99.12277 50.70005) (end 90.495301 59.327519) (width 0.25) (layer F.Cu) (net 11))
 (segment (start 70.937375 67.471301) (end 70.312699 66.846625) (width 0.25) (layer F.Cu) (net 11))
 (segment (start 157.94995 50.70005) (end 99.12277 50.70005) (width 0.25) (layer F.Cu) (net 11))
 (segment (start 82.524 57.8) (end 89.294 51.03) (width 0.25) (layer F.Cu) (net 11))
 (segment (start 73.91359 57.8) (end 82.524 57.8) (width 0.25) (layer F.Cu) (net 11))
 (segment (start 205.872003 37.824999) (end 195.247002 48.45) (width 0.25) (layer F.Cu) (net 10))
 (segment (start 217.984003 37.824999) (end 205.872003 37.824999) (width 0.25) (layer F.Cu) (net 10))
 (segment (start 222.609002 33.2) (end 217.984003 37.824999) (width 0.25) (layer F.Cu) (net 10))
 (segment (start 239.4 33.2) (end 222.609002 33.2) (width 0.25) (layer F.Cu) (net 10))
 (segment (start 195.247002 48.45) (end 190.8 48.45) (width 0.25) (layer F.Cu) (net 10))
 (segment (start 80.43401 57.34999) (end 86.754 51.03) (width 0.25) (layer F.Cu) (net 10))
 (segment (start 73.72719 57.34999) (end 80.43401 57.34999) (width 0.25) (layer F.Cu) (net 10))
 (segment (start 67.772699 63.304481) (end 73.72719 57.34999) (width 0.25) (layer F.Cu) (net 10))
 (segment (start 67.772699 66.846625) (end 67.772699 63.304481) (width 0.25) (layer F.Cu) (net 10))
 (segment (start 68.847385 67.921311) (end 67.772699 66.846625) (width 0.25) (layer F.Cu) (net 10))
 (segment (start 90.057025 67.921311) (end 68.847385 67.921311) (width 0.25) (layer F.Cu) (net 10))
 (segment (start 90.94531 67.033026) (end 90.057025 67.921311) (width 0.25) (layer F.Cu) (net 10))
 (segment (start 90.945311 59.513919) (end 90.94531 67.033026) (width 0.25) (layer F.Cu) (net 10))
 (segment (start 99.30917 51.15006) (end 90.945311 59.513919) (width 0.25) (layer F.Cu) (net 10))
 (segment (start 158.13635 51.15006) (end 99.30917 51.15006) (width 0.25) (layer F.Cu) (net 10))
 (segment (start 160.3864 48.90001) (end 158.13635 51.15006) (width 0.25) (layer F.Cu) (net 10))
 (segment (start 190.34999 48.90001) (end 160.3864 48.90001) (width 0.25) (layer F.Cu) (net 10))
 (segment (start 190.8 48.45) (end 190.34999 48.90001) (width 0.25) (layer F.Cu) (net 10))
 (segment (start 225.387999 37.824999) (end 214.762998 48.45) (width 0.25) (layer F.Cu) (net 9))
 (segment (start 236.884003 37.824999) (end 225.387999 37.824999) (width 0.25) (layer F.Cu) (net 9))
 (segment (start 241.509002 33.2) (end 236.884003 37.824999) (width 0.25) (layer F.Cu) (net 9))
 (segment (start 258.3 33.2) (end 241.509002 33.2) (width 0.25) (layer F.Cu) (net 9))
 (segment (start 214.762998 48.45) (end 197.1 48.45) (width 0.25) (layer F.Cu) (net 9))
 (via (at 91.8 45.9) (size 0.8) (drill 0.4) (layers F.Cu B.Cu) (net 9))
 (segment (start 105.925001 31.774999) (end 91.8 45.9) (width 0.25) (layer F.Cu) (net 9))
 (segment (start 240.084001 31.774999) (end 105.925001 31.774999) (width 0.25) (layer F.Cu) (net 9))
 (segment (start 240.825001 32.515999) (end 240.084001 31.774999) (width 0.25) (layer F.Cu) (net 9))
 (segment (start 240.084001 34.625001) (end 240.825001 33.884001) (width 0.25) (layer F.Cu) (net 9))
 (segment (start 238.715999 34.625001) (end 240.084001 34.625001) (width 0.25) (layer F.Cu) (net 9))
 (segment (start 237.741008 33.65001) (end 238.715999 34.625001) (width 0.25) (layer F.Cu) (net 9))
 (segment (start 222.795402 33.65001) (end 237.741008 33.65001) (width 0.25) (layer F.Cu) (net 9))
 (segment (start 207.995412 48.45) (end 222.795402 33.65001) (width 0.25) (layer F.Cu) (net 9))
 (segment (start 240.825001 33.884001) (end 240.825001 32.515999) (width 0.25) (layer F.Cu) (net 9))
 (segment (start 197.1 48.45) (end 207.995412 48.45) (width 0.25) (layer F.Cu) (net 9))
 (segment (start 91.8 45.9) (end 90.1 47.6) (width 0.25) (layer B.Cu) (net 9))
 (via (at 90 47.6) (size 0.8) (drill 0.4) (layers F.Cu B.Cu) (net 9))
 (segment (start 90.1 47.6) (end 90 47.6) (width 0.25) (layer B.Cu) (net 9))
 (segment (start 84.206588 51.03) (end 84.214 51.03) (width 0.25) (layer F.Cu) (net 9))
 (segment (start 67.874999 34.698411) (end 84.206588 51.03) (width 0.25) (layer F.Cu) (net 9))
 (segment (start 67.874999 32.515999) (end 67.874999 34.698411) (width 0.25) (layer F.Cu) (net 9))
 (segment (start 68.615999 31.774999) (end 67.874999 32.515999) (width 0.25) (layer F.Cu) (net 9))
 (segment (start 72.809334 31.774999) (end 68.615999 31.774999) (width 0.25) (layer F.Cu) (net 9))
 (segment (start 88.634335 47.6) (end 72.809334 31.774999) (width 0.25) (layer F.Cu) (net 9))
 (segment (start 90 47.6) (end 88.634335 47.6) (width 0.25) (layer F.Cu) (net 9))
 (segment (start 114.506552 60.952784) (end 94.747216 60.952784) (width 0.25) (layer F.Cu) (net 8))
 (segment (start 73.477375 49.828699) (end 80.472699 49.828699) (width 0.25) (layer F.Cu) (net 8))
 (segment (start 60.152699 64.294891) (end 72.852699 51.594891) (width 0.25) (layer F.Cu) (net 8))
 (segment (start 72.852699 50.453375) (end 73.477375 49.828699) (width 0.25) (layer F.Cu) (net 8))
 (segment (start 60.152699 67.406301) (end 60.152699 64.294891) (width 0.25) (layer F.Cu) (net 8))
 (segment (start 72.852699 51.594891) (end 72.852699 50.453375) (width 0.25) (layer F.Cu) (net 8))
 (segment (start 62.017739 69.271341) (end 60.152699 67.406301) (width 0.25) (layer F.Cu) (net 8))
 (segment (start 90.616225 69.271341) (end 62.017739 69.271341) (width 0.25) (layer F.Cu) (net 8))
 (segment (start 94.747216 65.14035) (end 90.616225 69.271341) (width 0.25) (layer F.Cu) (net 8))
 (segment (start 80.472699 49.828699) (end 81.674 51.03) (width 0.25) (layer F.Cu) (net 8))
 (segment (start 94.747216 60.952784) (end 94.747216 65.14035) (width 0.25) (layer F.Cu) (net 8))
 (segment (start 213.093448 61.802784) (end 201.440664 50.15) (width 0.25) (layer F.Cu) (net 7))
 (segment (start 182.6 50.15) (end 181.025011 51.724989) (width 0.25) (layer F.Cu) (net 7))
 (segment (start 201.440664 50.15) (end 182.6 50.15) (width 0.25) (layer F.Cu) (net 7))
 (segment (start 181.025011 51.724989) (end 118.525011 51.724989) (width 0.25) (layer F.Cu) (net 7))
 (segment (start 118.525011 51.724989) (end 111.6 58.65) (width 0.25) (layer F.Cu) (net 7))
 (segment (start 111.6 58.65) (end 96.3 58.65) (width 0.25) (layer F.Cu) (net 7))
 (segment (start 96.3 58.65) (end 95.4 58.65) (width 0.25) (layer F.Cu) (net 7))
 (via (at 95.4 58.65) (size 0.8) (drill 0.4) (layers F.Cu B.Cu) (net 7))
 (via (at 79.2 56.1) (size 0.8) (drill 0.4) (layers F.Cu B.Cu) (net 7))
 (segment (start 81.75 58.65) (end 79.2 56.1) (width 0.25) (layer B.Cu) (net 7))
 (segment (start 95.4 58.65) (end 81.75 58.65) (width 0.25) (layer B.Cu) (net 7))
 (segment (start 79.2 51.096) (end 79.134 51.03) (width 0.25) (layer F.Cu) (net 7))
 (segment (start 79.2 56.1) (end 79.2 51.096) (width 0.25) (layer F.Cu) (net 7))
 (segment (start 65.232699 66.846625) (end 65.232699 62.391301) (width 0.25) (layer F.Cu) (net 6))
 (segment (start 65.232699 62.391301) (end 76.594 51.03) (width 0.25) (layer F.Cu) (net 6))
 (segment (start 90.243425 68.371321) (end 66.757395 68.371321) (width 0.25) (layer F.Cu) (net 6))
 (segment (start 91.395319 67.219427) (end 90.243425 68.371321) (width 0.25) (layer F.Cu) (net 6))
 (segment (start 111.6 59.5) (end 91.59564 59.5) (width 0.25) (layer F.Cu) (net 6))
 (segment (start 91.39532 59.70032) (end 91.395319 67.219427) (width 0.25) (layer F.Cu) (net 6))
 (segment (start 91.59564 59.5) (end 91.39532 59.70032) (width 0.25) (layer F.Cu) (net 6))
 (segment (start 181.274999 52.174999) (end 118.925001 52.174999) (width 0.25) (layer F.Cu) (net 6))
 (segment (start 66.757395 68.371321) (end 65.232699 66.846625) (width 0.25) (layer F.Cu) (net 6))
 (segment (start 118.925001 52.174999) (end 111.6 59.5) (width 0.25) (layer F.Cu) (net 6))
 (segment (start 182.7 53.6) (end 181.274999 52.174999) (width 0.25) (layer F.Cu) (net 6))
 (via (at 70.2 73.95) (size 0.8) (drill 0.4) (layers F.Cu B.Cu) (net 21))
 (segment (start 70.2 70.036) (end 70.2 73.95) (width 0.25) (layer B.Cu) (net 21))
 (segment (start 66.434 66.27) (end 70.2 70.036) (width 0.25) (layer B.Cu) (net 21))
 (segment (start 68.05 73.95) (end 67.9 74.1) (width 0.25) (layer F.Cu) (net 21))
 (segment (start 70.2 73.95) (end 68.05 73.95) (width 0.25) (layer F.Cu) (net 21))
 (segment (start 67.9 74.1) (end 61.7 74.1) (width 0.25) (layer F.Cu) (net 21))
 (segment (start 62.692699 66.846625) (end 62.692699 62.391301) (width 0.25) (layer F.Cu) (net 5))
 (segment (start 91.845328 67.405828) (end 90.429825 68.821331) (width 0.25) (layer F.Cu) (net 5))
 (segment (start 111.6 60.35) (end 91.845329 60.35) (width 0.25) (layer F.Cu) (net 5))
 (segment (start 118.35 53.6) (end 111.6 60.35) (width 0.25) (layer F.Cu) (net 5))
 (segment (start 62.692699 62.391301) (end 74.054 51.03) (width 0.25) (layer F.Cu) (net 5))
 (segment (start 64.667405 68.821331) (end 62.692699 66.846625) (width 0.25) (layer F.Cu) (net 5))
 (segment (start 90.429825 68.821331) (end 64.667405 68.821331) (width 0.25) (layer F.Cu) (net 5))
 (segment (start 91.845329 60.35) (end 91.845328 67.405828) (width 0.25) (layer F.Cu) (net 5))
 (segment (start 144.9 53.6) (end 118.35 53.6) (width 0.25) (layer F.Cu) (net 5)))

